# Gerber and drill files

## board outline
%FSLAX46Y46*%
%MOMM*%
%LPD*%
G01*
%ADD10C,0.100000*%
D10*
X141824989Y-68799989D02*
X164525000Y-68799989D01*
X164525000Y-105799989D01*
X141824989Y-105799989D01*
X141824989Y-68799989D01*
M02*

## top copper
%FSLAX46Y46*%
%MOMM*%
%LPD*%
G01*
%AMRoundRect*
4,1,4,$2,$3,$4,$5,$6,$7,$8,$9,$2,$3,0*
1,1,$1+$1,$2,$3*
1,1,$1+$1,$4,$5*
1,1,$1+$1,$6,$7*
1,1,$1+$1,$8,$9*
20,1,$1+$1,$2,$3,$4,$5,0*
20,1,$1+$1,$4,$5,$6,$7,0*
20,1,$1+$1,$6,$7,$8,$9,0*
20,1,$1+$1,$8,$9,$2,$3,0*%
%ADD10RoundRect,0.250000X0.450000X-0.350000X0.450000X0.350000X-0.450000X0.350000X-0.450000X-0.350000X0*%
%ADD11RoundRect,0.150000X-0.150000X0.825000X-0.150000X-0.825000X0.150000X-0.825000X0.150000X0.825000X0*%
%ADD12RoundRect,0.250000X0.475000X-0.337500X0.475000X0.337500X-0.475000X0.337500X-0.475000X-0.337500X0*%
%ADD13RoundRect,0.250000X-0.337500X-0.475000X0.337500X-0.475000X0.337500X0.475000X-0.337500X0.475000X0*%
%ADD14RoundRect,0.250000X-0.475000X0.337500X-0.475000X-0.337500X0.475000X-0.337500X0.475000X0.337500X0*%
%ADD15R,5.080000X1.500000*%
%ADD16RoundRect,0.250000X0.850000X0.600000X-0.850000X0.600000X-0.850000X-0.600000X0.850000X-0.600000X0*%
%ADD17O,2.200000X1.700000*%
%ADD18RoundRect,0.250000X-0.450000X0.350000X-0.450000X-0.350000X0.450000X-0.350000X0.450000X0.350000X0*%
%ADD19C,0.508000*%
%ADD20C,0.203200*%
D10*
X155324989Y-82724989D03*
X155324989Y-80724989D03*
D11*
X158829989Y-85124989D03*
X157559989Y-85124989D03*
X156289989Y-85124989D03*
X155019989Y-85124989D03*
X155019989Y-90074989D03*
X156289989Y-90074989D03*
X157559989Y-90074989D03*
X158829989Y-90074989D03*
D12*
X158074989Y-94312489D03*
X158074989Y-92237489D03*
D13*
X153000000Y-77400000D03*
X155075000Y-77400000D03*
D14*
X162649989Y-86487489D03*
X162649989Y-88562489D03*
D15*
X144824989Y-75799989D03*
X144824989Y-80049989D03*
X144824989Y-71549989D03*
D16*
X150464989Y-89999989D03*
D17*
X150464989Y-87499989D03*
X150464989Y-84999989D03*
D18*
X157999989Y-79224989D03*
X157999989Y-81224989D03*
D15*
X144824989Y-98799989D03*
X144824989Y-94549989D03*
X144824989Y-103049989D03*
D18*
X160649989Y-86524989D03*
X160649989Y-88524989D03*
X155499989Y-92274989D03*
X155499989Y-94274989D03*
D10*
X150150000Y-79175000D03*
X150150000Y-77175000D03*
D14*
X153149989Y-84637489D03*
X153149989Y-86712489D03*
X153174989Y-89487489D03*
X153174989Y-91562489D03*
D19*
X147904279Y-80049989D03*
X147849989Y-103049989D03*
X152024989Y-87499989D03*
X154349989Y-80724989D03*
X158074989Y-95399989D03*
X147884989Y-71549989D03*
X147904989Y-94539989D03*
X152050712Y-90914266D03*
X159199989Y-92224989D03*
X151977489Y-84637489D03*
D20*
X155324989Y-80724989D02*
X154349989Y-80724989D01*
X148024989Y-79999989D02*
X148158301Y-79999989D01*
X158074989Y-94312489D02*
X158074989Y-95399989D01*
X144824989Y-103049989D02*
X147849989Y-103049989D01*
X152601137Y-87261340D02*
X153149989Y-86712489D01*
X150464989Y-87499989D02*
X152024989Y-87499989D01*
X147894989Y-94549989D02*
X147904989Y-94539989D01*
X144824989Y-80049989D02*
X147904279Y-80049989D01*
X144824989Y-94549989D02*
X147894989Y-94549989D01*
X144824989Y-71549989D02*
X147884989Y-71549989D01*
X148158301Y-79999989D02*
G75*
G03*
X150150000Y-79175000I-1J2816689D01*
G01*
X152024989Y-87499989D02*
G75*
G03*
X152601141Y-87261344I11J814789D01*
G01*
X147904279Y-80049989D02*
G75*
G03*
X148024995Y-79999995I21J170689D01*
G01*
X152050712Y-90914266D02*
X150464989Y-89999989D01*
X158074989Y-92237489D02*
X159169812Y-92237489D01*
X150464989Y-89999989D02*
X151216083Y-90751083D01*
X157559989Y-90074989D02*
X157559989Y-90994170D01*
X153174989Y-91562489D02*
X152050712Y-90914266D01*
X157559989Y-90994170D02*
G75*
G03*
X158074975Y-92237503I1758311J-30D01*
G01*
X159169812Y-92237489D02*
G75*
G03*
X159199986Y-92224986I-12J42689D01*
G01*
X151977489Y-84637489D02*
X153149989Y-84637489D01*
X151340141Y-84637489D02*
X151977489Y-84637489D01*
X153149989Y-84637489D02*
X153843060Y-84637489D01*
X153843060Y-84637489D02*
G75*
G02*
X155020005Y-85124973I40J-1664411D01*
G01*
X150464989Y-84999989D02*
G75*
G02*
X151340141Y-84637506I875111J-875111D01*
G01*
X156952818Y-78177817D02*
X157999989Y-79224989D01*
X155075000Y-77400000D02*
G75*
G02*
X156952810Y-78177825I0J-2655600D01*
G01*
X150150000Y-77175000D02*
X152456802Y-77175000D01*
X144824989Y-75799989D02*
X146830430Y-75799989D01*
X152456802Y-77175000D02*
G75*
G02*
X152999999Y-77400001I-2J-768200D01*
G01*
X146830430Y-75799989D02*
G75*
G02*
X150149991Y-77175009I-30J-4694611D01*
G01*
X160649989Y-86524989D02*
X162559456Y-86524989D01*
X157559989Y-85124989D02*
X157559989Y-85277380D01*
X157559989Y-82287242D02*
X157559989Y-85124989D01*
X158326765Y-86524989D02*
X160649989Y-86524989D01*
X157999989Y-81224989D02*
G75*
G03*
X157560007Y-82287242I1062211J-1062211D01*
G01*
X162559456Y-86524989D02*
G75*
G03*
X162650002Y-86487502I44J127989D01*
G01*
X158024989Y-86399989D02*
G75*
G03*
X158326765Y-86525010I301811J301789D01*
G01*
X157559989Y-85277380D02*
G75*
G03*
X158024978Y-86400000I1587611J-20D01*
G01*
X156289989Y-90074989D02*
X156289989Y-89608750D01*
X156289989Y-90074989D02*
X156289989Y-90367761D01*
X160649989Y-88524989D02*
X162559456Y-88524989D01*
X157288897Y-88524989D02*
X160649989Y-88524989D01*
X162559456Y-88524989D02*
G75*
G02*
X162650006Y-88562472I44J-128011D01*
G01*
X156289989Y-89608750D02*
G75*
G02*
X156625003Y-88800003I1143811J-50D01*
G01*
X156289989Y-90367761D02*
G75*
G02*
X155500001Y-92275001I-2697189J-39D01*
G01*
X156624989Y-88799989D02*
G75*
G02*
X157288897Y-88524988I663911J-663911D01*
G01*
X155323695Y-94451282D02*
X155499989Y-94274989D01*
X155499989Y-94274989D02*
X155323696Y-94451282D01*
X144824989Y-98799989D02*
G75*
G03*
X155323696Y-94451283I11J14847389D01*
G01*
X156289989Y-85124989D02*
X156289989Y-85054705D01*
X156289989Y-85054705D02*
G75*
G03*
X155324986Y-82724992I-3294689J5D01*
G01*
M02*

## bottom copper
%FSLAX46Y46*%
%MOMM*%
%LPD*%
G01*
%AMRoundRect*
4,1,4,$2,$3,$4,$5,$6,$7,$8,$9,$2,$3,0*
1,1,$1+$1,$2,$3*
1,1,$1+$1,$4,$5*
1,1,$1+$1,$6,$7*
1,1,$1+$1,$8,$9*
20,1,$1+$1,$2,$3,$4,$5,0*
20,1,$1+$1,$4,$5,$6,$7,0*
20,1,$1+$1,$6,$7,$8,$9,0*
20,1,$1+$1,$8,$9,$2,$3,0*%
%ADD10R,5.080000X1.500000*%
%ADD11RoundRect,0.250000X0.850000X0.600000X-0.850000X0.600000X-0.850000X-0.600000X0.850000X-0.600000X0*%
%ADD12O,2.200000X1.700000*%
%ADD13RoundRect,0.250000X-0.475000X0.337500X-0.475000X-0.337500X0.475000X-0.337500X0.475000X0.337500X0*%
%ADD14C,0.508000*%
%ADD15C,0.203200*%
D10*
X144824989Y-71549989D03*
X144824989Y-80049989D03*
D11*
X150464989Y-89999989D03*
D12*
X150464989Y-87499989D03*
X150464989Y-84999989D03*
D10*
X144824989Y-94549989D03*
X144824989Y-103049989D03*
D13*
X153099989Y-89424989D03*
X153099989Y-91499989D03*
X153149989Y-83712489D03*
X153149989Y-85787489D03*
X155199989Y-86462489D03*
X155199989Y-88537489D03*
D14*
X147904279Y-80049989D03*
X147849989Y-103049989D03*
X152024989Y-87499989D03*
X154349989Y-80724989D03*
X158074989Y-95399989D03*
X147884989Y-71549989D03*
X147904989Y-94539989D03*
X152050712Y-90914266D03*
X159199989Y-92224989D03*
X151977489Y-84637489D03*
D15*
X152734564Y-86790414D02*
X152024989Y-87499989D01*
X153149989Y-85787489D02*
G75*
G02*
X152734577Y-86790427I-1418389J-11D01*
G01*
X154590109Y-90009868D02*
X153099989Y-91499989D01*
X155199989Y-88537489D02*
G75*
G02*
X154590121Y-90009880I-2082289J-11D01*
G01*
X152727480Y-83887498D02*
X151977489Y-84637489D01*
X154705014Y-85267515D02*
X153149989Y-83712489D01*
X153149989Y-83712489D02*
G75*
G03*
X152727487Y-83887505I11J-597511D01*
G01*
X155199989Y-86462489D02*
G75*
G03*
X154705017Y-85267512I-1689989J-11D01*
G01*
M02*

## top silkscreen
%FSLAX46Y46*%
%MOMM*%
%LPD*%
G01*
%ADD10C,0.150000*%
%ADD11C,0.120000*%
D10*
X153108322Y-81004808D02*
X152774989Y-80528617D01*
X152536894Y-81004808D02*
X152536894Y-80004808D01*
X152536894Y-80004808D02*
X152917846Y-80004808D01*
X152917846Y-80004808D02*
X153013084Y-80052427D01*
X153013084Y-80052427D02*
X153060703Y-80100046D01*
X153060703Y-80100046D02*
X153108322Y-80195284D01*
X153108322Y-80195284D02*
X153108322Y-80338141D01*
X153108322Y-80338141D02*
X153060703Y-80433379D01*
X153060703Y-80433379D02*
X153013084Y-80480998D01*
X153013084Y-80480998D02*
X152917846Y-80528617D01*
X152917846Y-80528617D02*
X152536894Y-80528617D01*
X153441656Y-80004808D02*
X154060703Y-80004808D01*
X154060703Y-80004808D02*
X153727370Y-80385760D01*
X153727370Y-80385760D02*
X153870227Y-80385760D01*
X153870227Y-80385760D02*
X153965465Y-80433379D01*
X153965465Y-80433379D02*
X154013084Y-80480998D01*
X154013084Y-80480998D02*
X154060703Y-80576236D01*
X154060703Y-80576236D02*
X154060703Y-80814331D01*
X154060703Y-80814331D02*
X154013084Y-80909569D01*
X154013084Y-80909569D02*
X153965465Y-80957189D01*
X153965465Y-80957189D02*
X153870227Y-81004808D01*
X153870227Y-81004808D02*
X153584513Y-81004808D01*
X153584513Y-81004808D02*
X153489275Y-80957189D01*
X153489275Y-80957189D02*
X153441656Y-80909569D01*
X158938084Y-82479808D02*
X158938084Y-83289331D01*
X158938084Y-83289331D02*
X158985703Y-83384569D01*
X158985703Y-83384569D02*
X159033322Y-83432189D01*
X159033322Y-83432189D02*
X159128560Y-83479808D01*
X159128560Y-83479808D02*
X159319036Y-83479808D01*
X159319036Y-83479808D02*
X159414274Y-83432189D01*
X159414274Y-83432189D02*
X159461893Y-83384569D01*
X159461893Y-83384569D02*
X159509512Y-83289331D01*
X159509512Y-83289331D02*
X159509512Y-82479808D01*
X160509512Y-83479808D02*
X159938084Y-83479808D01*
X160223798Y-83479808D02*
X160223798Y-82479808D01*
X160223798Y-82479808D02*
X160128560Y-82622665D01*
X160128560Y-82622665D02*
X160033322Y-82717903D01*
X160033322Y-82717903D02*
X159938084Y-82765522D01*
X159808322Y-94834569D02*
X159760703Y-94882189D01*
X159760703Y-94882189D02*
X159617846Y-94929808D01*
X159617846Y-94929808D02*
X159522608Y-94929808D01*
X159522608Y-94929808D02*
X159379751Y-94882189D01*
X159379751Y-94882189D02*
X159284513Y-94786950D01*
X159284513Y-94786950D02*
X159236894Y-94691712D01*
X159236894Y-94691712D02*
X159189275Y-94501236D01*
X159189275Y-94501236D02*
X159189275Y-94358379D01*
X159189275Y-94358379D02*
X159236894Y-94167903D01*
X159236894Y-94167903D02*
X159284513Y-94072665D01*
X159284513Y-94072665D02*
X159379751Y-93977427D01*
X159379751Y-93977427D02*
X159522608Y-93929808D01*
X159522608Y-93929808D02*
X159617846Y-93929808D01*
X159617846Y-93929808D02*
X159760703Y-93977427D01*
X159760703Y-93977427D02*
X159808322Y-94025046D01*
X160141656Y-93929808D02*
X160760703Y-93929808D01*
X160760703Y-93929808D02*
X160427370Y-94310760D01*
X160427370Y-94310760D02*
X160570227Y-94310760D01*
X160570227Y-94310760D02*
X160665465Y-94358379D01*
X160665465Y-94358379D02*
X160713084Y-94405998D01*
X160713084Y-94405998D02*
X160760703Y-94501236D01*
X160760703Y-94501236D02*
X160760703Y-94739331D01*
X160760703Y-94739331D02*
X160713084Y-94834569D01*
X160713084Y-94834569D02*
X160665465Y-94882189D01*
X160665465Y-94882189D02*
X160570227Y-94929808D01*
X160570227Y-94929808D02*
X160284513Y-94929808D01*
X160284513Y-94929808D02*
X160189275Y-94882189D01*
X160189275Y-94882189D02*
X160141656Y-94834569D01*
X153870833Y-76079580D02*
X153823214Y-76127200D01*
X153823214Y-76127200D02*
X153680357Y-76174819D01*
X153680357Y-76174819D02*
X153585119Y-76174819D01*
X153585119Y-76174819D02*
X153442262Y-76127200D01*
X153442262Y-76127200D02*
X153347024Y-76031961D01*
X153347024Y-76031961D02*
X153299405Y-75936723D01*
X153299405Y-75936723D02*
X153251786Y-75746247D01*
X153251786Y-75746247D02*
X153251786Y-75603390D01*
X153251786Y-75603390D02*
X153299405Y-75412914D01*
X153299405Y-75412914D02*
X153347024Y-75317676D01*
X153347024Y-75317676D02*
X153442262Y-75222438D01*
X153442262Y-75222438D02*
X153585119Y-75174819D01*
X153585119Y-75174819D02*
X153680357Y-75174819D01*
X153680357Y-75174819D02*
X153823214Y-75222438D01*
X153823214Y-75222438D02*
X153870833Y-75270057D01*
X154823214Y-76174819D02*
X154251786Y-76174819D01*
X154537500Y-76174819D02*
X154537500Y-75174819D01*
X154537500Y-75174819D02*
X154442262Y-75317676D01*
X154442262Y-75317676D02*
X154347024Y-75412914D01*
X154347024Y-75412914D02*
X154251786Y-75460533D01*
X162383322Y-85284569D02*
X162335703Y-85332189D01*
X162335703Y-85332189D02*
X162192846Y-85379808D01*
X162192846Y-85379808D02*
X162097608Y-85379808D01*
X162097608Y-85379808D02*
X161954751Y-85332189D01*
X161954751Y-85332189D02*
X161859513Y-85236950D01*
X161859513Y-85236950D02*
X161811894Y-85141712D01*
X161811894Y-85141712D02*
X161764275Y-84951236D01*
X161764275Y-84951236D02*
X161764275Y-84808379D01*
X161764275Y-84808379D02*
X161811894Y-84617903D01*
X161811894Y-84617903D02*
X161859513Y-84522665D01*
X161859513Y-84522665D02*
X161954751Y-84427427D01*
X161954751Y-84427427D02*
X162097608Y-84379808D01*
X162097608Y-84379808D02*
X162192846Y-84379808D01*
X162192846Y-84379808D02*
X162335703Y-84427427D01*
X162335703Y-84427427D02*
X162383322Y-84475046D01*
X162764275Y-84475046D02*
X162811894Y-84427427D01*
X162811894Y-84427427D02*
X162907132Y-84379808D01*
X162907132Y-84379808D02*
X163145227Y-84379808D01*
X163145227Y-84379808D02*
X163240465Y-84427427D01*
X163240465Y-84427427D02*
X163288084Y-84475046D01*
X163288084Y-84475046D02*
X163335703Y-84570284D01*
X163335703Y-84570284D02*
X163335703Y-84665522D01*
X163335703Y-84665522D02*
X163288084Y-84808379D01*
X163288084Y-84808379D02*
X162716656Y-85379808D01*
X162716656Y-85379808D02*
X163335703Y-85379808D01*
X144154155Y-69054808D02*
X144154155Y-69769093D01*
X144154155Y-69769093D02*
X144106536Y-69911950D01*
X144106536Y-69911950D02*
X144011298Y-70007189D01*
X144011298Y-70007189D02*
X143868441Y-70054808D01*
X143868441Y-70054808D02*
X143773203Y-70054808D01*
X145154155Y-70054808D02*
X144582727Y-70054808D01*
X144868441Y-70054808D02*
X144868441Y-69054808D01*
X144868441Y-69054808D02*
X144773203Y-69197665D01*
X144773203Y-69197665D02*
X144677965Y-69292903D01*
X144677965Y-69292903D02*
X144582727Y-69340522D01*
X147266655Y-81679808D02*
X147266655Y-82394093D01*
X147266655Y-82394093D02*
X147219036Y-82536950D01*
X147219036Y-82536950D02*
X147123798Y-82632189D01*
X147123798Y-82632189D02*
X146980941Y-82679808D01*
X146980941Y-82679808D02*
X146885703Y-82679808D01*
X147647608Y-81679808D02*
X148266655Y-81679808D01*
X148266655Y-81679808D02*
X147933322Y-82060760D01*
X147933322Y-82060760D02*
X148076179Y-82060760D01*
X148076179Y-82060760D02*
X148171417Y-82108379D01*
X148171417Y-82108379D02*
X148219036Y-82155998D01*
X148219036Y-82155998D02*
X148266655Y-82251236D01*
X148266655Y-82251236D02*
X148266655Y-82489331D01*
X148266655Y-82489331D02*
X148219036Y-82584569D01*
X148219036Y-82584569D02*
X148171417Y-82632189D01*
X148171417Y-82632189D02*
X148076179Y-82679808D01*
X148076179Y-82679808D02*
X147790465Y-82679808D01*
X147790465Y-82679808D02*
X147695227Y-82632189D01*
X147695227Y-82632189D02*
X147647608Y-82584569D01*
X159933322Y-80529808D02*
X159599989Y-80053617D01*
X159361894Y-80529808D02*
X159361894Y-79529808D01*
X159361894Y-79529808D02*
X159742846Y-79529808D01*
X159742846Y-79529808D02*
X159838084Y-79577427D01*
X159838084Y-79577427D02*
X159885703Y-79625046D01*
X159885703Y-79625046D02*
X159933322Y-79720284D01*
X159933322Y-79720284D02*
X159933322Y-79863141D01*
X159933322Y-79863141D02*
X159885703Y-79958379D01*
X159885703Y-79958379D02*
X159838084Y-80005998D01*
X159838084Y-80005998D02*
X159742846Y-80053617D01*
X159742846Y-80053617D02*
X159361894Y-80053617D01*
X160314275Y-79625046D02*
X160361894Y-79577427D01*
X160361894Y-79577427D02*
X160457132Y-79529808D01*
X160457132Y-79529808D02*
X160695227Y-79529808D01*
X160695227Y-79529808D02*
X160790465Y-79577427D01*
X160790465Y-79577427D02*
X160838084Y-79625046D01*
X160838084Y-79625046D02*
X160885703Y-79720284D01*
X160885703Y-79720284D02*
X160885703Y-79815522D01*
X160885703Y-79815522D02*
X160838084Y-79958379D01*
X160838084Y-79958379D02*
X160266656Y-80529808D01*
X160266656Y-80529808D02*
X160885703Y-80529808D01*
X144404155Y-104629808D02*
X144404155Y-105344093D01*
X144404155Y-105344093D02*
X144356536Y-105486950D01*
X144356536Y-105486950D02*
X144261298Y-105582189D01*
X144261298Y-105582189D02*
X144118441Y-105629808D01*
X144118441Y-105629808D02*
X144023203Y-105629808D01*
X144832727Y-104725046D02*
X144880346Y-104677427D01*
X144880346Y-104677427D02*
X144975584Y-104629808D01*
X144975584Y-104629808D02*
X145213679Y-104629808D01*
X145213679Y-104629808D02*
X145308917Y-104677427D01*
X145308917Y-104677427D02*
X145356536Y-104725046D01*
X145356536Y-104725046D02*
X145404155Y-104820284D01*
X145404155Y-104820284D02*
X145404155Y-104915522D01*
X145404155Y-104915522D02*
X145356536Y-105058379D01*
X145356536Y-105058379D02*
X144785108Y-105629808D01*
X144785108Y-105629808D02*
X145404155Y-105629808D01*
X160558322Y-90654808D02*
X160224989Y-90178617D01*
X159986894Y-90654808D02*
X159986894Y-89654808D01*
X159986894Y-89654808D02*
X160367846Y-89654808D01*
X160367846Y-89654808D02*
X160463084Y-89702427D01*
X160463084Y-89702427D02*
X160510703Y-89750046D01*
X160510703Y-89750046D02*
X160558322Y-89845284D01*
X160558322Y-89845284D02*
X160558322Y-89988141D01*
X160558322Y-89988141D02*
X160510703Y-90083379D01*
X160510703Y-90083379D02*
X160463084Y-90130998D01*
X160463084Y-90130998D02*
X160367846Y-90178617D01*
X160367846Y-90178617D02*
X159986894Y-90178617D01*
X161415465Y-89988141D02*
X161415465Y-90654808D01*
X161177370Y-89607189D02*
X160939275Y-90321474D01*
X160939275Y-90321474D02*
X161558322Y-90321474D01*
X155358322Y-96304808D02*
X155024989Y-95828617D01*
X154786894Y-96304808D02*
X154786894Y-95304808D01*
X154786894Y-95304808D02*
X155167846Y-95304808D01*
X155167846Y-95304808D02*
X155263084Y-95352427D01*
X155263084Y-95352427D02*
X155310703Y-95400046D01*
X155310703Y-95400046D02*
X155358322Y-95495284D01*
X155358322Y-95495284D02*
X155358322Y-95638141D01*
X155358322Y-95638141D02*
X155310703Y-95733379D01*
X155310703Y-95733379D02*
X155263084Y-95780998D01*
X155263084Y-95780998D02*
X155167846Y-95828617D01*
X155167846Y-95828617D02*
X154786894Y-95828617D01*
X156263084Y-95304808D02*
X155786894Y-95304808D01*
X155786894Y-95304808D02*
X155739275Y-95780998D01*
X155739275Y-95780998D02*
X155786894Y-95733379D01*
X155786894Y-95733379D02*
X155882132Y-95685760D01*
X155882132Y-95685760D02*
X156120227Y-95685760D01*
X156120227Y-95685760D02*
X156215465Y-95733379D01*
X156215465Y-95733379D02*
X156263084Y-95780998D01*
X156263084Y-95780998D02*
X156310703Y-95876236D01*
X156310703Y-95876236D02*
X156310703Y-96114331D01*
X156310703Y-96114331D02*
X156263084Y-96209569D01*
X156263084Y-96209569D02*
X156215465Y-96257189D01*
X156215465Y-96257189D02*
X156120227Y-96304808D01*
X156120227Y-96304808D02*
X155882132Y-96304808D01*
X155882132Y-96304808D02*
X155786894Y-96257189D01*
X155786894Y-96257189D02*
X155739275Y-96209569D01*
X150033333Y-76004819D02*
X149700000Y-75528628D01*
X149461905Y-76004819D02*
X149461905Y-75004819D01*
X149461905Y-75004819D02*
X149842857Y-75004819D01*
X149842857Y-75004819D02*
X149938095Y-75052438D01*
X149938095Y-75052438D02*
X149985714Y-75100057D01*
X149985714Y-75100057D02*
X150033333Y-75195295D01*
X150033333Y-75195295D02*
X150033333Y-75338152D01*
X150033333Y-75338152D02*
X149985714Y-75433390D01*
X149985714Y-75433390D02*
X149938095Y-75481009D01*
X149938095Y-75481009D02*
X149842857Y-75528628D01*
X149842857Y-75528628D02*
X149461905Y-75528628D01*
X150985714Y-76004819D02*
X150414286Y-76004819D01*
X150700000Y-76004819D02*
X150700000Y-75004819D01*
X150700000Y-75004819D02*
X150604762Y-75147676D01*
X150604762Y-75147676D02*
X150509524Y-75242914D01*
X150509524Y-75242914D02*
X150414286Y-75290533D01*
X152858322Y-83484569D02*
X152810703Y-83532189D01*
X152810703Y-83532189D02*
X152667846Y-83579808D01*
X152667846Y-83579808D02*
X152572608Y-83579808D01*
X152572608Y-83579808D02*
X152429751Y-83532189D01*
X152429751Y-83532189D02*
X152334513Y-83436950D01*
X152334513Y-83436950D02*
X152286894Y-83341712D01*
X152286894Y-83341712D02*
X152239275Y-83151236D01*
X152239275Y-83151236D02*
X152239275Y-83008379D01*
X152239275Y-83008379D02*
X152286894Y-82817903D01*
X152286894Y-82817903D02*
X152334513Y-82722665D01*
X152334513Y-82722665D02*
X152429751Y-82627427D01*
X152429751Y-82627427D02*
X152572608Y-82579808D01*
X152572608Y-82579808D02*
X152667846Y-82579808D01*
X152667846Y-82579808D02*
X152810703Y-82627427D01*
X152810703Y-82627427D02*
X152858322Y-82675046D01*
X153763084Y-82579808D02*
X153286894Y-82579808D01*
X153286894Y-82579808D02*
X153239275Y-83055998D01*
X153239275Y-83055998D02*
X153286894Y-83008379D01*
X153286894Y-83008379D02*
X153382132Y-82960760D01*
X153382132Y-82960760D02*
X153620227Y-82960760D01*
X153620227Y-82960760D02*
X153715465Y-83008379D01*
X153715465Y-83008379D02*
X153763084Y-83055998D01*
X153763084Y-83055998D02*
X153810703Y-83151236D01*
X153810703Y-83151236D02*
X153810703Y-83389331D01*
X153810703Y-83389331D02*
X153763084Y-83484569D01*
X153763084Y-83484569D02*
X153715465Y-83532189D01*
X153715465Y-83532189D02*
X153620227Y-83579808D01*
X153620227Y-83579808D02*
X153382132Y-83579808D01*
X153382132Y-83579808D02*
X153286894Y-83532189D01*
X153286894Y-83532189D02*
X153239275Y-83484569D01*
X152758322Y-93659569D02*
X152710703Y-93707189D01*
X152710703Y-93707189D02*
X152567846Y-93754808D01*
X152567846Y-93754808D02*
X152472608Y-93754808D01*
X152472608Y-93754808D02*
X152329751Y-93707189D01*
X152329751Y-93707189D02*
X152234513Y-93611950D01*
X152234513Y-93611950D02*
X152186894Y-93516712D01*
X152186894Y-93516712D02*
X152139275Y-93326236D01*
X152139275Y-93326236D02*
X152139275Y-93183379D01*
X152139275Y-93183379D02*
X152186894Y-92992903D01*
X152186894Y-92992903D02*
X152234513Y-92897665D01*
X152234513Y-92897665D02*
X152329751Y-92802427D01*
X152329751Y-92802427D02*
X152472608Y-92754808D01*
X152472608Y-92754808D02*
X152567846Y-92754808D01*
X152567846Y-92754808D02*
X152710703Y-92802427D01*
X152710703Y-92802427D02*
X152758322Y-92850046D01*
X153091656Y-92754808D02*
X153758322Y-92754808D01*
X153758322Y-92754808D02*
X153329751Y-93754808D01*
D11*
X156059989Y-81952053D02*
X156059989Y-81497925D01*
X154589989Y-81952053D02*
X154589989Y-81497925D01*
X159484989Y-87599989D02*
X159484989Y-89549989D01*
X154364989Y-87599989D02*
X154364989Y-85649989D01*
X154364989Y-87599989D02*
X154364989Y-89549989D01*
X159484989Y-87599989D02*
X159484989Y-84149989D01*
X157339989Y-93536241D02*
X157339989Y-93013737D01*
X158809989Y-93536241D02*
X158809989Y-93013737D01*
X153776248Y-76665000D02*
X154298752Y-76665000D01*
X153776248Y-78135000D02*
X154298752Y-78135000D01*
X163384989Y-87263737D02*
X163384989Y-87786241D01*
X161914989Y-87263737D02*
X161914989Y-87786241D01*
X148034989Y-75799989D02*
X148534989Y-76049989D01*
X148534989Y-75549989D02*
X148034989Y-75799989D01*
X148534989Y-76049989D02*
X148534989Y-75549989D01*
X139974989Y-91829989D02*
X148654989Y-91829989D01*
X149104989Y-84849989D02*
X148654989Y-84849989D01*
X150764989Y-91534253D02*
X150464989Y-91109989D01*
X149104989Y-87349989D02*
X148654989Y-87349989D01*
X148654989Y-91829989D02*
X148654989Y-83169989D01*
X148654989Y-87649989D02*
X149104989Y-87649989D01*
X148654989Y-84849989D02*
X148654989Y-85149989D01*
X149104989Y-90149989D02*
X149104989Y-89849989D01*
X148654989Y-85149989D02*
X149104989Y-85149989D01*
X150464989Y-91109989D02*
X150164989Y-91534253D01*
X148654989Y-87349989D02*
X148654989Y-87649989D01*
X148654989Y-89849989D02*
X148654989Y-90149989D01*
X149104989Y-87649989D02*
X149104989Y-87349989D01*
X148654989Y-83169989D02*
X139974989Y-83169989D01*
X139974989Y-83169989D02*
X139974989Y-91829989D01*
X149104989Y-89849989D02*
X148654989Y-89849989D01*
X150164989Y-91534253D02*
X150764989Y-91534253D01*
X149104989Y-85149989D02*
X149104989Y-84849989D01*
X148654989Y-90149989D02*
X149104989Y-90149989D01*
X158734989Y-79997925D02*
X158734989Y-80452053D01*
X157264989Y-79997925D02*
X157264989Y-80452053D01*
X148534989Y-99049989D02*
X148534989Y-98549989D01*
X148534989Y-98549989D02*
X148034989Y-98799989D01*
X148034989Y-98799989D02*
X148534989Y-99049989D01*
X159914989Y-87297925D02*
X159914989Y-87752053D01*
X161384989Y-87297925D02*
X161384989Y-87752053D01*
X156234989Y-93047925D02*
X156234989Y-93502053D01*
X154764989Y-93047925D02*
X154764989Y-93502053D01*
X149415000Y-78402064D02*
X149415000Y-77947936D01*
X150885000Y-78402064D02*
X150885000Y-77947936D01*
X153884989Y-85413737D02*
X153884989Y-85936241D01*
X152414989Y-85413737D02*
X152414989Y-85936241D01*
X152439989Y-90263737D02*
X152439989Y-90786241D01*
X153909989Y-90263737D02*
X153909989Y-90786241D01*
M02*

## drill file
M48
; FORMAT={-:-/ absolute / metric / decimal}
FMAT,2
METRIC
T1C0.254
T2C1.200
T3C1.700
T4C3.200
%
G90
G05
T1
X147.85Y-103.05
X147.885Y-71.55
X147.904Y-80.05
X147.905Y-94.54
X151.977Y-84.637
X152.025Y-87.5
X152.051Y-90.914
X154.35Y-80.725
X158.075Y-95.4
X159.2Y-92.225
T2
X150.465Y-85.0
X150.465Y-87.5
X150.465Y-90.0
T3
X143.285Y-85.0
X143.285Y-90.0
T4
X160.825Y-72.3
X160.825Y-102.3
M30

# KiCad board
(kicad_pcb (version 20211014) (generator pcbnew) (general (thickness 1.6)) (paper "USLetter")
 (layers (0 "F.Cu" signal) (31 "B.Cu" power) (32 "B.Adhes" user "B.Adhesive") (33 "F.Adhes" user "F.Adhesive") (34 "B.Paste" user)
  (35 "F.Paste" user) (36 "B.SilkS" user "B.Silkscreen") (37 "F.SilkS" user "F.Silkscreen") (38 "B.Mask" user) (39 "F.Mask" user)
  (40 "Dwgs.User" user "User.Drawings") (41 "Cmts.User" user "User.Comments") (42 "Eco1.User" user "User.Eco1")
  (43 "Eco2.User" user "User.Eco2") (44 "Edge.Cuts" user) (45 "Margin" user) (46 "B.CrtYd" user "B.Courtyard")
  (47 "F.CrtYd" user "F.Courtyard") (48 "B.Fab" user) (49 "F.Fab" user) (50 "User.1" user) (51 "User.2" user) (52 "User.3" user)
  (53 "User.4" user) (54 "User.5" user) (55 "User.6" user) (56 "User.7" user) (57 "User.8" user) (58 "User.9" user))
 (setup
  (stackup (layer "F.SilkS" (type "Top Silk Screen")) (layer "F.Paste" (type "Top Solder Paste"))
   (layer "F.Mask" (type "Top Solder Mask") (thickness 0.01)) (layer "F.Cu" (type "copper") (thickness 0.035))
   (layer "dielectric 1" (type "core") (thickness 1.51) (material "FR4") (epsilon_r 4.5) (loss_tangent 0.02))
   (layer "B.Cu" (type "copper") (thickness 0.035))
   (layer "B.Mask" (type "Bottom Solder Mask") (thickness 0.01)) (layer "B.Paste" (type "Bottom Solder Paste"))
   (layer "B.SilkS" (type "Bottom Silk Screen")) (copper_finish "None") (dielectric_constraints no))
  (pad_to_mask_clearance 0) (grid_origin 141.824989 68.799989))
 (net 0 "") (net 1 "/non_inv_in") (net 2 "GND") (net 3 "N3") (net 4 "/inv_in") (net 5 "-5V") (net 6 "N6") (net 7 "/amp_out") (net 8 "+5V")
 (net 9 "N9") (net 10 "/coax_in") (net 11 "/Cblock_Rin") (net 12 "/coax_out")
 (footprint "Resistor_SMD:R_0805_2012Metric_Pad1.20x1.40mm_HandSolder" (layer "F.Cu") (at 155.324989 81.724989 90)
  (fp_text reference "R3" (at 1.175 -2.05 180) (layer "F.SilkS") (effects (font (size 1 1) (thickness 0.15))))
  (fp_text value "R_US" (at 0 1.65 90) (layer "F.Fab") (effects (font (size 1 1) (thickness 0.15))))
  (fp_line (start -0.227064 0.735) (end 0.227064 0.735) (layer "F.SilkS") (width 0.12))
  (fp_line (start -0.227064 -0.735) (end 0.227064 -0.735) (layer "F.SilkS") (width 0.12))
  (pad "1" smd roundrect (at -1 0 90) (size 1.2 1.4) (layers "F.Cu" "F.Paste" "F.Mask") (roundrect_rratio 0.208333) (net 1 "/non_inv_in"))
  (pad "2" smd roundrect (at 1 0 90) (size 1.2 1.4) (layers "F.Cu" "F.Paste" "F.Mask") (roundrect_rratio 0.208333) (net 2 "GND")))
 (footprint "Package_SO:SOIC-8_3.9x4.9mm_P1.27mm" (layer "F.Cu") (at 156.924989 87.599989 -90)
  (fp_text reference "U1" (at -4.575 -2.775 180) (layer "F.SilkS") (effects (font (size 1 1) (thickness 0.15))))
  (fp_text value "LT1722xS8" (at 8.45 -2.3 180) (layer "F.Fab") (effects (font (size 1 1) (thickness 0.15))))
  (fp_line (start 0 -2.56) (end 1.95 -2.56) (layer "F.SilkS") (width 0.12))
  (fp_line (start 0 2.56) (end -1.95 2.56) (layer "F.SilkS") (width 0.12))
  (fp_line (start 0 2.56) (end 1.95 2.56) (layer "F.SilkS") (width 0.12))
  (fp_line (start 0 -2.56) (end -3.45 -2.56) (layer "F.SilkS") (width 0.12))
  (pad "1" smd roundrect (at -2.475 -1.905 270) (size 1.95 0.6) (layers "F.Cu" "F.Paste" "F.Mask") (roundrect_rratio 0.25) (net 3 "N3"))
  (pad "2" smd roundrect (at -2.475 -0.635 270) (size 1.95 0.6) (layers "F.Cu" "F.Paste" "F.Mask") (roundrect_rratio 0.25) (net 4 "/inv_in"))
  (pad "3" smd roundrect (at -2.475 0.635 270) (size 1.95 0.6) (layers "F.Cu" "F.Paste" "F.Mask") (roundrect_rratio 0.25)
   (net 1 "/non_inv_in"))
  (pad "4" smd roundrect (at -2.475 1.905 270) (size 1.95 0.6) (layers "F.Cu" "F.Paste" "F.Mask") (roundrect_rratio 0.25) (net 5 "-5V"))
  (pad "5" smd roundrect (at 2.475 1.905 270) (size 1.95 0.6) (layers "F.Cu" "F.Paste" "F.Mask") (roundrect_rratio 0.25) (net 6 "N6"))
  (pad "6" smd roundrect (at 2.475 0.635 270) (size 1.95 0.6) (layers "F.Cu" "F.Paste" "F.Mask") (roundrect_rratio 0.25) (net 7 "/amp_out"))
  (pad "7" smd roundrect (at 2.475 -0.635 270) (size 1.95 0.6) (layers "F.Cu" "F.Paste" "F.Mask") (roundrect_rratio 0.25) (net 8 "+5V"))
  (pad "8" smd roundrect (at 2.475 -1.905 270) (size 1.95 0.6) (layers "F.Cu" "F.Paste" "F.Mask") (roundrect_rratio 0.25) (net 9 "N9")))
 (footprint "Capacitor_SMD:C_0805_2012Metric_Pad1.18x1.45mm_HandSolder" (layer "F.Cu") (at 158.074989 93.274989 90)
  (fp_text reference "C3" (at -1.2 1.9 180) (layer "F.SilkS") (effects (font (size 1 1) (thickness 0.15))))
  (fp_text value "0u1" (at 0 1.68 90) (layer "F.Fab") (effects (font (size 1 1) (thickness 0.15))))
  (fp_line (start -0.261252 -0.735) (end 0.261252 -0.735) (layer "F.SilkS") (width 0.12))
  (fp_line (start -0.261252 0.735) (end 0.261252 0.735) (layer "F.SilkS") (width 0.12))
  (pad "1" smd roundrect (at -1.0375 0 90) (size 1.175 1.45) (layers "F.Cu" "F.Paste" "F.Mask") (roundrect_rratio 0.212766) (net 2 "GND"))
  (pad "2" smd roundrect (at 1.0375 0 90) (size 1.175 1.45) (layers "F.Cu" "F.Paste" "F.Mask") (roundrect_rratio 0.212766) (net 8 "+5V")))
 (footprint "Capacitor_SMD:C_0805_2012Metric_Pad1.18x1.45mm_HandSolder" (layer "F.Cu") (at 154.0375 77.4)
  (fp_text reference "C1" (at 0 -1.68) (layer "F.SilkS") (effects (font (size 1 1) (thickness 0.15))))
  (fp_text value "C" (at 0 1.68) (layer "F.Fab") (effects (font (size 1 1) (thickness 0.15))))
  (fp_line (start -0.261252 -0.735) (end 0.261252 -0.735) (layer "F.SilkS") (width 0.12))
  (fp_line (start -0.261252 0.735) (end 0.261252 0.735) (layer "F.SilkS") (width 0.12))
  (pad "1" smd roundrect (at -1.0375 0) (size 1.175 1.45) (layers "F.Cu" "F.Paste" "F.Mask") (roundrect_rratio 0.212766) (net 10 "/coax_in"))
  (pad "2" smd roundrect (at 1.0375 0) (size 1.175 1.45) (layers "F.Cu" "F.Paste" "F.Mask") (roundrect_rratio 0.212766)
   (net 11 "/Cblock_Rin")))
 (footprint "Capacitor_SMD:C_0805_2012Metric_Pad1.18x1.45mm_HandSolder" (layer "F.Cu") (at 162.649989 87.524989 -90)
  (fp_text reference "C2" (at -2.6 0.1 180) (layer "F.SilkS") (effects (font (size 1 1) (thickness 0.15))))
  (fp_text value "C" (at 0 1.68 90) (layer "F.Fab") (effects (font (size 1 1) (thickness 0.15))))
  (fp_line (start -0.261252 -0.735) (end 0.261252 -0.735) (layer "F.SilkS") (width 0.12))
  (fp_line (start -0.261252 0.735) (end 0.261252 0.735) (layer "F.SilkS") (width 0.12))
  (pad "1" smd roundrect (at -1.0375 0 270) (size 1.175 1.45) (layers "F.Cu" "F.Paste" "F.Mask") (roundrect_rratio 0.212766)
   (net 4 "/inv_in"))
  (pad "2" smd roundrect (at 1.0375 0 270) (size 1.175 1.45) (layers "F.Cu" "F.Paste" "F.Mask") (roundrect_rratio 0.212766)
   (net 7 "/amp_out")))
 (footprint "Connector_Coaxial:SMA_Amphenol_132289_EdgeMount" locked (layer "F.Cu") (at 144.824989 75.799989 180)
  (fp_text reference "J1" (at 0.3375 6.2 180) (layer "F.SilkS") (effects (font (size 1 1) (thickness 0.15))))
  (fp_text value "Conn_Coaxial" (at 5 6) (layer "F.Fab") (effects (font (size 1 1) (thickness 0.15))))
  (fp_line (start -3.21 0) (end -3.71 -0.25) (layer "F.SilkS") (width 0.12))
  (fp_line (start -3.71 0.25) (end -3.21 0) (layer "F.SilkS") (width 0.12))
  (fp_line (start -3.71 -0.25) (end -3.71 0.25) (layer "F.SilkS") (width 0.12))
  (pad "1" smd rect locked (at 0 0 270) (size 1.5 5.08) (layers "F.Cu" "F.Paste" "F.Mask") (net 10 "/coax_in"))
  (pad "2" smd rect locked (at 0 -4.25 270) (size 1.5 5.08) (layers "F.Cu" "F.Paste" "F.Mask") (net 2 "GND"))
  (pad "2" smd rect locked (at 0 4.25 270) (size 1.5 5.08) (layers "B.Cu" "B.Paste" "B.Mask") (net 2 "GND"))
  (pad "2" smd rect locked (at 0 -4.25 270) (size 1.5 5.08) (layers "B.Cu" "B.Paste" "B.Mask") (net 2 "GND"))
  (pad "2" smd rect locked (at 0 4.25 270) (size 1.5 5.08) (layers "F.Cu" "F.Paste" "F.Mask") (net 2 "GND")))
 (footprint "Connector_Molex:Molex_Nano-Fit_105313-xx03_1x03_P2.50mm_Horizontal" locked (layer "F.Cu") (at 150.464989 89.999989 180)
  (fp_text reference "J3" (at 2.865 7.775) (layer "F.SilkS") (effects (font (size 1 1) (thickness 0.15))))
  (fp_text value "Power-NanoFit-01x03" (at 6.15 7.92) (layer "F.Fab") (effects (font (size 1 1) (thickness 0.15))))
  (fp_line (start 10.49 -1.83) (end 1.81 -1.83) (layer "F.SilkS") (width 0.12))
  (fp_line (start 1.36 5.15) (end 1.81 5.15) (layer "F.SilkS") (width 0.12))
  (fp_line (start -0.3 -1.534264) (end 0 -1.11) (layer "F.SilkS") (width 0.12))
  (fp_line (start 1.36 2.65) (end 1.81 2.65) (layer "F.SilkS") (width 0.12))
  (fp_line (start 1.81 -1.83) (end 1.81 6.83) (layer "F.SilkS") (width 0.12))
  (fp_line (start 1.81 2.35) (end 1.36 2.35) (layer "F.SilkS") (width 0.12))
  (fp_line (start 1.81 5.15) (end 1.81 4.85) (layer "F.SilkS") (width 0.12))
  (fp_line (start 1.36 -0.15) (end 1.36 0.15) (layer "F.SilkS") (width 0.12))
  (fp_line (start 1.81 4.85) (end 1.36 4.85) (layer "F.SilkS") (width 0.12))
  (fp_line (start 0 -1.11) (end 0.3 -1.534264) (layer "F.SilkS") (width 0.12))
  (fp_line (start 1.81 2.65) (end 1.81 2.35) (layer "F.SilkS") (width 0.12))
  (fp_line (start 1.81 0.15) (end 1.81 -0.15) (layer "F.SilkS") (width 0.12))
  (fp_line (start 1.36 2.35) (end 1.36 2.65) (layer "F.SilkS") (width 0.12))
  (fp_line (start 1.81 6.83) (end 10.49 6.83) (layer "F.SilkS") (width 0.12))
  (fp_line (start 10.49 6.83) (end 10.49 -1.83) (layer "F.SilkS") (width 0.12))
  (fp_line (start 1.36 0.15) (end 1.81 0.15) (layer "F.SilkS") (width 0.12))
  (fp_line (start 0.3 -1.534264) (end -0.3 -1.534264) (layer "F.SilkS") (width 0.12))
  (fp_line (start 1.36 4.85) (end 1.36 5.15) (layer "F.SilkS") (width 0.12))
  (fp_line (start 1.81 -0.15) (end 1.36 -0.15) (layer "F.SilkS") (width 0.12))
  (pad "" np_thru_hole circle locked (at 7.18 0 180) (size 1.7 1.7) (drill 1.7) (layers *.Cu *.Mask))
  (pad "" np_thru_hole circle locked (at 7.18 5 180) (size 1.7 1.7) (drill 1.7) (layers *.Cu *.Mask))
  (pad "1" thru_hole roundrect locked (at 0 0 180) (size 2.2 1.7) (drill 1.2) (layers *.Cu *.Mask) (roundrect_rratio 0.147059) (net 8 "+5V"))
  (pad "2" thru_hole oval locked (at 0 2.5 180) (size 2.2 1.7) (drill 1.2) (layers *.Cu *.Mask) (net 2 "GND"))
  (pad "3" thru_hole oval locked (at 0 5 180) (size 2.2 1.7) (drill 1.2) (layers *.Cu *.Mask) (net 5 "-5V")))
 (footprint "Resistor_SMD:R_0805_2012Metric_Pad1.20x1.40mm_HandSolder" (layer "F.Cu") (at 157.999989 80.224989 -90)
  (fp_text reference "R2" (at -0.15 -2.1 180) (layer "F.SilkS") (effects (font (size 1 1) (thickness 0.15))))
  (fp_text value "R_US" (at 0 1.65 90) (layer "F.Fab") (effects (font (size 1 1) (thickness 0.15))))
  (fp_line (start -0.227064 -0.735) (end 0.227064 -0.735) (layer "F.SilkS") (width 0.12))
  (fp_line (start -0.227064 0.735) (end 0.227064 0.735) (layer "F.SilkS") (width 0.12))
  (pad "1" smd roundrect (at -1 0 270) (size 1.2 1.4) (layers "F.Cu" "F.Paste" "F.Mask") (roundrect_rratio 0.208333) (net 11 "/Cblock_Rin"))
  (pad "2" smd roundrect (at 1 0 270) (size 1.2 1.4) (layers "F.Cu" "F.Paste" "F.Mask") (roundrect_rratio 0.208333) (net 4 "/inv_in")))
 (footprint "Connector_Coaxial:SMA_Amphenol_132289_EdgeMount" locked (layer "F.Cu") (at 144.824989 98.799989 180)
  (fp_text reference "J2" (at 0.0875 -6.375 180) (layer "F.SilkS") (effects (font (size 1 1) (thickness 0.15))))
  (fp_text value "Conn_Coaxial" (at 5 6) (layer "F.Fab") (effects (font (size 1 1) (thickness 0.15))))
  (fp_line (start -3.71 -0.25) (end -3.71 0.25) (layer "F.SilkS") (width 0.12))
  (fp_line (start -3.71 0.25) (end -3.21 0) (layer "F.SilkS") (width 0.12))
  (fp_line (start -3.21 0) (end -3.71 -0.25) (layer "F.SilkS") (width 0.12))
  (pad "1" smd rect locked (at 0 0 270) (size 1.5 5.08) (layers "F.Cu" "F.Paste" "F.Mask") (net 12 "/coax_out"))
  (pad "2" smd rect locked (at 0 4.25 270) (size 1.5 5.08) (layers "B.Cu" "B.Paste" "B.Mask") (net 2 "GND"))
  (pad "2" smd rect locked (at 0 4.25 270) (size 1.5 5.08) (layers "F.Cu" "F.Paste" "F.Mask") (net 2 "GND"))
  (pad "2" smd rect locked (at 0 -4.25 270) (size 1.5 5.08) (layers "B.Cu" "B.Paste" "B.Mask") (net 2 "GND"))
  (pad "2" smd rect locked (at 0 -4.25 270) (size 1.5 5.08) (layers "F.Cu" "F.Paste" "F.Mask") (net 2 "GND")))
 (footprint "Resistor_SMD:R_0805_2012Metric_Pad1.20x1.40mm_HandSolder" (layer "F.Cu") (at 160.649989 87.524989 -90)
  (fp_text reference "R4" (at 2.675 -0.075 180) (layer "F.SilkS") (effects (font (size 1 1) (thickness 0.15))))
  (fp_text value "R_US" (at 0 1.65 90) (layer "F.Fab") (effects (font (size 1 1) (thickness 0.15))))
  (fp_line (start -0.227064 0.735) (end 0.227064 0.735) (layer "F.SilkS") (width 0.12))
  (fp_line (start -0.227064 -0.735) (end 0.227064 -0.735) (layer "F.SilkS") (width 0.12))
  (pad "1" smd roundrect (at -1 0 270) (size 1.2 1.4) (layers "F.Cu" "F.Paste" "F.Mask") (roundrect_rratio 0.208333) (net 4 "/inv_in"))
  (pad "2" smd roundrect (at 1 0 270) (size 1.2 1.4) (layers "F.Cu" "F.Paste" "F.Mask") (roundrect_rratio 0.208333) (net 7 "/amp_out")))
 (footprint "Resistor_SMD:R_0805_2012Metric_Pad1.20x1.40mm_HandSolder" (layer "F.Cu") (at 155.499989 93.274989 -90)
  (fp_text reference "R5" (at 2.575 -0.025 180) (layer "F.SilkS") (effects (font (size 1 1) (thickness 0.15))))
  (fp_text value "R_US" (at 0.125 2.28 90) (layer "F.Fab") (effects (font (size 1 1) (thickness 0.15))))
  (fp_line (start -0.227064 -0.735) (end 0.227064 -0.735) (layer "F.SilkS") (width 0.12))
  (fp_line (start -0.227064 0.735) (end 0.227064 0.735) (layer "F.SilkS") (width 0.12))
  (pad "1" smd roundrect (at -1 0 270) (size 1.2 1.4) (layers "F.Cu" "F.Paste" "F.Mask") (roundrect_rratio 0.208333) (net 7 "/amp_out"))
  (pad "2" smd roundrect (at 1 0 270) (size 1.2 1.4) (layers "F.Cu" "F.Paste" "F.Mask") (roundrect_rratio 0.208333) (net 12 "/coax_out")))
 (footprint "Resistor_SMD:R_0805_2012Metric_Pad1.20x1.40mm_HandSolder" (layer "F.Cu") (at 150.15 78.175 90)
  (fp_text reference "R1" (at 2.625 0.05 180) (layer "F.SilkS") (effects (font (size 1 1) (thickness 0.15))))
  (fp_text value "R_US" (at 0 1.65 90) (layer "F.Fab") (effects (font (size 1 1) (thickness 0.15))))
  (fp_line (start -0.227064 -0.735) (end 0.227064 -0.735) (layer "F.SilkS") (width 0.12))
  (fp_line (start -0.227064 0.735) (end 0.227064 0.735) (layer "F.SilkS") (width 0.12))
  (pad "1" smd roundrect (at -1 0 90) (size 1.2 1.4) (layers "F.Cu" "F.Paste" "F.Mask") (roundrect_rratio 0.208333) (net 2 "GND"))
  (pad "2" smd roundrect (at 1 0 90) (size 1.2 1.4) (layers "F.Cu" "F.Paste" "F.Mask") (roundrect_rratio 0.208333) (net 10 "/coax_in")))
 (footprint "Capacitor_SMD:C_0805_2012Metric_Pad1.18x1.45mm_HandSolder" (layer "F.Cu") (at 153.149989 85.674989 -90)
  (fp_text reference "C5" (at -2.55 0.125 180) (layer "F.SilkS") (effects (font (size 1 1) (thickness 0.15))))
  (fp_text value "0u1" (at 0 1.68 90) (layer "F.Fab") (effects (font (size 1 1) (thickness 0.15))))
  (fp_line (start -0.261252 -0.735) (end 0.261252 -0.735) (layer "F.SilkS") (width 0.12))
  (fp_line (start -0.261252 0.735) (end 0.261252 0.735) (layer "F.SilkS") (width 0.12))
  (pad "1" smd roundrect (at -1.0375 0 270) (size 1.175 1.45) (layers "F.Cu" "F.Paste" "F.Mask") (roundrect_rratio 0.212766) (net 5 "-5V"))
  (pad "2" smd roundrect (at 1.0375 0 270) (size 1.175 1.45) (layers "F.Cu" "F.Paste" "F.Mask") (roundrect_rratio 0.212766) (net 2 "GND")))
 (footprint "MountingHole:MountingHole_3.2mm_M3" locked (layer "F.Cu") (at 160.824989 72.299989)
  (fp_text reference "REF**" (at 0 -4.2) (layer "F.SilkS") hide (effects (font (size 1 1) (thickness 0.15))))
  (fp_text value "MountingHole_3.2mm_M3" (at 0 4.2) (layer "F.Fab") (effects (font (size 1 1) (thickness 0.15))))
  (pad "" np_thru_hole circle locked (at 0 0) (size 3.2 3.2) (drill 3.2) (layers *.Cu *.Mask)))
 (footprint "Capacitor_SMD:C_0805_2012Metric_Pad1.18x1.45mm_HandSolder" (layer "F.Cu") (at 153.174989 90.524989 -90)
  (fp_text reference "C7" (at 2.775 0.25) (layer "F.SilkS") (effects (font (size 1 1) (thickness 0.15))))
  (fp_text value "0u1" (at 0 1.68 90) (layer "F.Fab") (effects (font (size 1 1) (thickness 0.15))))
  (fp_line (start -0.261252 0.735) (end 0.261252 0.735) (layer "F.SilkS") (width 0.12))
  (fp_line (start -0.261252 -0.735) (end 0.261252 -0.735) (layer "F.SilkS") (width 0.12))
  (pad "1" smd roundrect (at -1.0375 0 270) (size 1.175 1.45) (layers "F.Cu" "F.Paste" "F.Mask") (roundrect_rratio 0.212766) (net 5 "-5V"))
  (pad "2" smd roundrect (at 1.0375 0 270) (size 1.175 1.45) (layers "F.Cu" "F.Paste" "F.Mask") (roundrect_rratio 0.212766) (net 8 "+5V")))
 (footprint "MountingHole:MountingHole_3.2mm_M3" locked (layer "F.Cu") (at 160.824989 102.299989)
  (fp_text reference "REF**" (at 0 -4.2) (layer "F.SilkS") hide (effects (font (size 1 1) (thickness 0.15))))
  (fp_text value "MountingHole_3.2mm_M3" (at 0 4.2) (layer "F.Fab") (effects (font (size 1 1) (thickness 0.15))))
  (pad "" np_thru_hole circle locked (at 0 0) (size 3.2 3.2) (drill 3.2) (layers F&B.Cu *.Mask)))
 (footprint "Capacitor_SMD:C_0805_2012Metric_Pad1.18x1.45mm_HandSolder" (layer "B.Cu") (at 153.099989 90.462489 -90)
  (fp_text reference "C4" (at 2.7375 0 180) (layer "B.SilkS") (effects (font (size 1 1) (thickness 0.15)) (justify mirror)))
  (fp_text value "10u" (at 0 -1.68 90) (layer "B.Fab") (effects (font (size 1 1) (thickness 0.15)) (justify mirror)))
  (pad "1" smd roundrect (at -1.0375 0 270) (size 1.175 1.45) (layers "B.Cu" "B.Paste" "B.Mask") (roundrect_rratio 0.212766) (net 2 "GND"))
  (pad "2" smd roundrect (at 1.0375 0 270) (size 1.175 1.45) (layers "B.Cu" "B.Paste" "B.Mask") (roundrect_rratio 0.212766) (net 8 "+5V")))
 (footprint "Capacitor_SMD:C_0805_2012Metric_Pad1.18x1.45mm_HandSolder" (layer "B.Cu") (at 153.149989 84.749989 -90)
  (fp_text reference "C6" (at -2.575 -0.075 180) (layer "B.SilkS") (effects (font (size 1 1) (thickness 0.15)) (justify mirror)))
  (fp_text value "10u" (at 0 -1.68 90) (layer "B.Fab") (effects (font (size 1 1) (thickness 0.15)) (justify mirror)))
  (pad "1" smd roundrect (at -1.0375 0 270) (size 1.175 1.45) (layers "B.Cu" "B.Paste" "B.Mask") (roundrect_rratio 0.212766) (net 5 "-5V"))
  (pad "2" smd roundrect (at 1.0375 0 270) (size 1.175 1.45) (layers "B.Cu" "B.Paste" "B.Mask") (roundrect_rratio 0.212766) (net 2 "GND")))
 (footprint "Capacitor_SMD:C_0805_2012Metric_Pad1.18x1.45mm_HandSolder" (layer "B.Cu") (at 155.199989 87.499989 -90)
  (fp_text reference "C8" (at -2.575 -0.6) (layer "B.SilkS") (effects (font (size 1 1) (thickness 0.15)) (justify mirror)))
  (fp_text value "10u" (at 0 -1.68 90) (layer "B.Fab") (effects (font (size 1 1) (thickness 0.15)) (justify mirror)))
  (pad "1" smd roundrect (at -1.0375 0 270) (size 1.175 1.45) (layers "B.Cu" "B.Paste" "B.Mask") (roundrect_rratio 0.212766) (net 5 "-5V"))
  (pad "2" smd roundrect (at 1.0375 0 270) (size 1.175 1.45) (layers "B.Cu" "B.Paste" "B.Mask") (roundrect_rratio 0.212766) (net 8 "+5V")))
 (gr_rect locked (start 141.824989 68.799989) (end 164.525 105.799989) (layer "Edge.Cuts") (width 0.1) (fill none))
 (segment (start 155.324989 80.724989) (end 154.349989 80.724989) (width 0.2032) (layer "F.Cu") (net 2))
 (segment (start 148.024989 79.999989) (end 148.158301 79.999989) (width 0.2032) (layer "F.Cu") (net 2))
 (segment (start 158.074989 94.312489) (end 158.074989 95.399989) (width 0.2032) (layer "F.Cu") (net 2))
 (segment (start 144.824989 103.049989) (end 147.849989 103.049989) (width 0.2032) (layer "F.Cu") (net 2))
 (segment (start 152.601137 87.26134) (end 153.149989 86.712489) (width 0.2032) (layer "F.Cu") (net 2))
 (segment (start 150.464989 87.499989) (end 152.024989 87.499989) (width 0.2032) (layer "F.Cu") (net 2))
 (segment (start 147.894989 94.549989) (end 147.904989 94.539989) (width 0.2032) (layer "F.Cu") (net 2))
 (segment (start 144.824989 80.049989) (end 147.904279 80.049989) (width 0.2032) (layer "F.Cu") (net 2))
 (segment (start 144.824989 94.549989) (end 147.894989 94.549989) (width 0.2032) (layer "F.Cu") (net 2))
 (segment (start 144.824989 71.549989) (end 147.884989 71.549989) (width 0.2032) (layer "F.Cu") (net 2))
 (via (at 147.904279 80.049989) (size 0.508) (drill 0.254) (layers "F.Cu" "B.Cu") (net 2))
 (via (at 147.849989 103.049989) (size 0.508) (drill 0.254) (layers "F.Cu" "B.Cu") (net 2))
 (via (at 152.024989 87.499989) (size 0.508) (drill 0.254) (layers "F.Cu" "B.Cu") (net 2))
 (via (at 154.349989 80.724989) (size 0.508) (drill 0.254) (layers "F.Cu" "B.Cu") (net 2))
 (via (at 158.074989 95.399989) (size 0.508) (drill 0.254) (layers "F.Cu" "B.Cu") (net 2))
 (via (at 147.884989 71.549989) (size 0.508) (drill 0.254) (layers "F.Cu" "B.Cu") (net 2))
 (via (at 147.904989 94.539989) (size 0.508) (drill 0.254) (layers "F.Cu" "B.Cu") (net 2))
 (arc (start 148.158301 79.999989) (mid 149.236201 79.785581) (end 150.15 79.175) (width 0.2032) (layer "F.Cu") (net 2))
 (arc (start 152.024989 87.499989) (mid 152.336798 87.437966) (end 152.601137 87.26134) (width 0.2032) (layer "F.Cu") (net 2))
 (arc (start 147.904279 80.049989) (mid 147.969607 80.036994) (end 148.024989 79.999989) (width 0.2032) (layer "F.Cu") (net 2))
 (segment (start 152.734564 86.790414) (end 152.024989 87.499989) (width 0.2032) (layer "B.Cu") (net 2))
 (arc (start 153.149989 85.787489) (mid 153.042024 86.330268) (end 152.734564 86.790414) (width 0.2032) (layer "B.Cu") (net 2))
 (segment (start 152.050712 90.914266) (end 150.464989 89.999989) (width 0.2032) (layer "F.Cu") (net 8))
 (segment (start 158.074989 92.237489) (end 159.169812 92.237489) (width 0.2032) (layer "F.Cu") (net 8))
 (segment (start 150.464989 89.999989) (end 151.216083 90.751083) (width 0.2032) (layer "F.Cu") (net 8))
 (segment (start 157.559989 90.074989) (end 157.559989 90.99417) (width 0.2032) (layer "F.Cu") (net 8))
 (segment (start 153.174989 91.562489) (end 152.050712 90.914266) (width 0.2032) (layer "F.Cu") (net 8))
 (via (at 152.050712 90.914266) (size 0.508) (drill 0.254) (layers "F.Cu" "B.Cu") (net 8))
 (via (at 159.199989 92.224989) (size 0.508) (drill 0.254) (layers "F.Cu" "B.Cu") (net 8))
 (arc (start 157.559989 90.99417) (mid 157.693833 91.667049) (end 158.074989 92.237489) (width 0.2032) (layer "F.Cu") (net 8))
 (arc (start 159.169812 92.237489) (mid 159.186144 92.23424) (end 159.199989 92.224989) (width 0.2032) (layer "F.Cu") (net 8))
 (segment (start 154.590109 90.009868) (end 153.099989 91.499989) (width 0.2032) (layer "B.Cu") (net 8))
 (arc (start 155.199989 88.537489) (mid 155.041486 89.334335) (end 154.590109 90.009868) (width 0.2032) (layer "B.Cu") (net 8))
 (segment (start 151.977489 84.637489) (end 153.149989 84.637489) (width 0.2032) (layer "F.Cu") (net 5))
 (segment (start 151.340141 84.637489) (end 151.977489 84.637489) (width 0.2032) (layer "F.Cu") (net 5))
 (segment (start 153.149989 84.637489) (end 153.84306 84.637489) (width 0.2032) (layer "F.Cu") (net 5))
 (via (at 151.977489 84.637489) (size 0.508) (drill 0.254) (layers "F.Cu" "B.Cu") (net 5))
 (arc (start 153.84306 84.637489) (mid 154.480009 84.764186) (end 155.019989 85.124989) (width 0.2032) (layer "F.Cu") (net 5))
 (arc (start 150.464989 84.999989) (mid 150.866512 84.7317) (end 151.340141 84.637489) (width 0.2032) (layer "F.Cu") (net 5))
 (segment (start 152.72748 83.887498) (end 151.977489 84.637489) (width 0.2032) (layer "B.Cu") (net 5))
 (segment (start 154.705014 85.267515) (end 153.149989 83.712489) (width 0.2032) (layer "B.Cu") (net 5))
 (arc (start 153.149989 83.712489) (mid 152.921329 83.757972) (end 152.72748 83.887498) (width 0.2032) (layer "B.Cu") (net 5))
 (arc (start 155.199989 86.462489) (mid 155.071349 85.815774) (end 154.705014 85.267515) (width 0.2032) (layer "B.Cu") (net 5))
 (segment (start 156.952818 78.177817) (end 157.999989 79.224989) (width 0.2032) (layer "F.Cu") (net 11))
 (arc (start 155.075 77.4) (mid 156.091268 77.602148) (end 156.952818 78.177817) (width 0.2032) (layer "F.Cu") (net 11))
 (segment (start 150.15 77.175) (end 152.456802 77.175) (width 0.2032) (layer "F.Cu") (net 10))
 (segment (start 144.824989 75.799989) (end 146.83043 75.799989) (width 0.2032) (layer "F.Cu") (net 10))
 (arc (start 152.456802 77.175) (mid 152.750778 77.233476) (end 153 77.4) (width 0.2032) (layer "F.Cu") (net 10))
 (arc (start 146.83043 75.799989) (mid 148.626968 76.157343) (end 150.15 77.175) (width 0.2032) (layer "F.Cu") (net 10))
 (segment (start 160.649989 86.524989) (end 162.559456 86.524989) (width 0.2032) (layer "F.Cu") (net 4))
 (segment (start 157.559989 85.124989) (end 157.559989 85.27738) (width 0.2032) (layer "F.Cu") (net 4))
 (segment (start 157.559989 82.287242) (end 157.559989 85.124989) (width 0.2032) (layer "F.Cu") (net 4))
 (segment (start 158.326765 86.524989) (end 160.649989 86.524989) (width 0.2032) (layer "F.Cu") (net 4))
 (arc (start 157.999989 81.224989) (mid 157.674341 81.712354) (end 157.559989 82.287242) (width 0.2032) (layer "F.Cu") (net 4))
 (arc (start 162.559456 86.524989) (mid 162.608452 86.515243) (end 162.649989 86.487489) (width 0.2032) (layer "F.Cu") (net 4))
 (arc (start 158.024989 86.399989) (mid 158.163445 86.492502) (end 158.326765 86.524989) (width 0.2032) (layer "F.Cu") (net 4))
 (arc (start 157.559989 85.27738) (mid 157.680839 85.884931) (end 158.024989 86.399989) (width 0.2032) (layer "F.Cu") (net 4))
 (segment (start 156.289989 90.074989) (end 156.289989 89.60875) (width 0.2032) (layer "F.Cu") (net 7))
 (segment (start 156.289989 90.074989) (end 156.289989 90.367761) (width 0.2032) (layer "F.Cu") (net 7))
 (segment (start 160.649989 88.524989) (end 162.559456 88.524989) (width 0.2032) (layer "F.Cu") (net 7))
 (segment (start 157.288897 88.524989) (end 160.649989 88.524989) (width 0.2032) (layer "F.Cu") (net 7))
 (arc (start 162.559456 88.524989) (mid 162.608452 88.534735) (end 162.649989 88.562489) (width 0.2032) (layer "F.Cu") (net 7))
 (arc (start 156.289989 89.60875) (mid 156.377053 89.171052) (end 156.624989 88.799989) (width 0.2032) (layer "F.Cu") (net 7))
 (arc (start 156.289989 90.367761) (mid 156.084674 91.399945) (end 155.499989 92.274989) (width 0.2032) (layer "F.Cu") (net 7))
 (arc (start 156.624989 88.799989) (mid 156.929592 88.596459) (end 157.288897 88.524989) (width 0.2032) (layer "F.Cu") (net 7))
 (segment (start 155.323695 94.451282) (end 155.499989 94.274989) (width 0.2032) (layer "F.Cu") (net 12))
 (segment (start 155.499989 94.274989) (end 155.323696 94.451282) (width 0.2032) (layer "F.Cu") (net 12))
 (arc (start 144.824989 98.799989) (mid 150.506848 97.669797) (end 155.323695 94.451282) (width 0.2032) (layer "F.Cu") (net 12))
 (segment (start 156.289989 85.124989) (end 156.289989 85.054705) (width 0.2032) (layer "F.Cu") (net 1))
 (arc (start 156.289989 85.054705) (mid 156.039194 83.793872) (end 155.324989 82.724989) (width 0.2032) (layer "F.Cu") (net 1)))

